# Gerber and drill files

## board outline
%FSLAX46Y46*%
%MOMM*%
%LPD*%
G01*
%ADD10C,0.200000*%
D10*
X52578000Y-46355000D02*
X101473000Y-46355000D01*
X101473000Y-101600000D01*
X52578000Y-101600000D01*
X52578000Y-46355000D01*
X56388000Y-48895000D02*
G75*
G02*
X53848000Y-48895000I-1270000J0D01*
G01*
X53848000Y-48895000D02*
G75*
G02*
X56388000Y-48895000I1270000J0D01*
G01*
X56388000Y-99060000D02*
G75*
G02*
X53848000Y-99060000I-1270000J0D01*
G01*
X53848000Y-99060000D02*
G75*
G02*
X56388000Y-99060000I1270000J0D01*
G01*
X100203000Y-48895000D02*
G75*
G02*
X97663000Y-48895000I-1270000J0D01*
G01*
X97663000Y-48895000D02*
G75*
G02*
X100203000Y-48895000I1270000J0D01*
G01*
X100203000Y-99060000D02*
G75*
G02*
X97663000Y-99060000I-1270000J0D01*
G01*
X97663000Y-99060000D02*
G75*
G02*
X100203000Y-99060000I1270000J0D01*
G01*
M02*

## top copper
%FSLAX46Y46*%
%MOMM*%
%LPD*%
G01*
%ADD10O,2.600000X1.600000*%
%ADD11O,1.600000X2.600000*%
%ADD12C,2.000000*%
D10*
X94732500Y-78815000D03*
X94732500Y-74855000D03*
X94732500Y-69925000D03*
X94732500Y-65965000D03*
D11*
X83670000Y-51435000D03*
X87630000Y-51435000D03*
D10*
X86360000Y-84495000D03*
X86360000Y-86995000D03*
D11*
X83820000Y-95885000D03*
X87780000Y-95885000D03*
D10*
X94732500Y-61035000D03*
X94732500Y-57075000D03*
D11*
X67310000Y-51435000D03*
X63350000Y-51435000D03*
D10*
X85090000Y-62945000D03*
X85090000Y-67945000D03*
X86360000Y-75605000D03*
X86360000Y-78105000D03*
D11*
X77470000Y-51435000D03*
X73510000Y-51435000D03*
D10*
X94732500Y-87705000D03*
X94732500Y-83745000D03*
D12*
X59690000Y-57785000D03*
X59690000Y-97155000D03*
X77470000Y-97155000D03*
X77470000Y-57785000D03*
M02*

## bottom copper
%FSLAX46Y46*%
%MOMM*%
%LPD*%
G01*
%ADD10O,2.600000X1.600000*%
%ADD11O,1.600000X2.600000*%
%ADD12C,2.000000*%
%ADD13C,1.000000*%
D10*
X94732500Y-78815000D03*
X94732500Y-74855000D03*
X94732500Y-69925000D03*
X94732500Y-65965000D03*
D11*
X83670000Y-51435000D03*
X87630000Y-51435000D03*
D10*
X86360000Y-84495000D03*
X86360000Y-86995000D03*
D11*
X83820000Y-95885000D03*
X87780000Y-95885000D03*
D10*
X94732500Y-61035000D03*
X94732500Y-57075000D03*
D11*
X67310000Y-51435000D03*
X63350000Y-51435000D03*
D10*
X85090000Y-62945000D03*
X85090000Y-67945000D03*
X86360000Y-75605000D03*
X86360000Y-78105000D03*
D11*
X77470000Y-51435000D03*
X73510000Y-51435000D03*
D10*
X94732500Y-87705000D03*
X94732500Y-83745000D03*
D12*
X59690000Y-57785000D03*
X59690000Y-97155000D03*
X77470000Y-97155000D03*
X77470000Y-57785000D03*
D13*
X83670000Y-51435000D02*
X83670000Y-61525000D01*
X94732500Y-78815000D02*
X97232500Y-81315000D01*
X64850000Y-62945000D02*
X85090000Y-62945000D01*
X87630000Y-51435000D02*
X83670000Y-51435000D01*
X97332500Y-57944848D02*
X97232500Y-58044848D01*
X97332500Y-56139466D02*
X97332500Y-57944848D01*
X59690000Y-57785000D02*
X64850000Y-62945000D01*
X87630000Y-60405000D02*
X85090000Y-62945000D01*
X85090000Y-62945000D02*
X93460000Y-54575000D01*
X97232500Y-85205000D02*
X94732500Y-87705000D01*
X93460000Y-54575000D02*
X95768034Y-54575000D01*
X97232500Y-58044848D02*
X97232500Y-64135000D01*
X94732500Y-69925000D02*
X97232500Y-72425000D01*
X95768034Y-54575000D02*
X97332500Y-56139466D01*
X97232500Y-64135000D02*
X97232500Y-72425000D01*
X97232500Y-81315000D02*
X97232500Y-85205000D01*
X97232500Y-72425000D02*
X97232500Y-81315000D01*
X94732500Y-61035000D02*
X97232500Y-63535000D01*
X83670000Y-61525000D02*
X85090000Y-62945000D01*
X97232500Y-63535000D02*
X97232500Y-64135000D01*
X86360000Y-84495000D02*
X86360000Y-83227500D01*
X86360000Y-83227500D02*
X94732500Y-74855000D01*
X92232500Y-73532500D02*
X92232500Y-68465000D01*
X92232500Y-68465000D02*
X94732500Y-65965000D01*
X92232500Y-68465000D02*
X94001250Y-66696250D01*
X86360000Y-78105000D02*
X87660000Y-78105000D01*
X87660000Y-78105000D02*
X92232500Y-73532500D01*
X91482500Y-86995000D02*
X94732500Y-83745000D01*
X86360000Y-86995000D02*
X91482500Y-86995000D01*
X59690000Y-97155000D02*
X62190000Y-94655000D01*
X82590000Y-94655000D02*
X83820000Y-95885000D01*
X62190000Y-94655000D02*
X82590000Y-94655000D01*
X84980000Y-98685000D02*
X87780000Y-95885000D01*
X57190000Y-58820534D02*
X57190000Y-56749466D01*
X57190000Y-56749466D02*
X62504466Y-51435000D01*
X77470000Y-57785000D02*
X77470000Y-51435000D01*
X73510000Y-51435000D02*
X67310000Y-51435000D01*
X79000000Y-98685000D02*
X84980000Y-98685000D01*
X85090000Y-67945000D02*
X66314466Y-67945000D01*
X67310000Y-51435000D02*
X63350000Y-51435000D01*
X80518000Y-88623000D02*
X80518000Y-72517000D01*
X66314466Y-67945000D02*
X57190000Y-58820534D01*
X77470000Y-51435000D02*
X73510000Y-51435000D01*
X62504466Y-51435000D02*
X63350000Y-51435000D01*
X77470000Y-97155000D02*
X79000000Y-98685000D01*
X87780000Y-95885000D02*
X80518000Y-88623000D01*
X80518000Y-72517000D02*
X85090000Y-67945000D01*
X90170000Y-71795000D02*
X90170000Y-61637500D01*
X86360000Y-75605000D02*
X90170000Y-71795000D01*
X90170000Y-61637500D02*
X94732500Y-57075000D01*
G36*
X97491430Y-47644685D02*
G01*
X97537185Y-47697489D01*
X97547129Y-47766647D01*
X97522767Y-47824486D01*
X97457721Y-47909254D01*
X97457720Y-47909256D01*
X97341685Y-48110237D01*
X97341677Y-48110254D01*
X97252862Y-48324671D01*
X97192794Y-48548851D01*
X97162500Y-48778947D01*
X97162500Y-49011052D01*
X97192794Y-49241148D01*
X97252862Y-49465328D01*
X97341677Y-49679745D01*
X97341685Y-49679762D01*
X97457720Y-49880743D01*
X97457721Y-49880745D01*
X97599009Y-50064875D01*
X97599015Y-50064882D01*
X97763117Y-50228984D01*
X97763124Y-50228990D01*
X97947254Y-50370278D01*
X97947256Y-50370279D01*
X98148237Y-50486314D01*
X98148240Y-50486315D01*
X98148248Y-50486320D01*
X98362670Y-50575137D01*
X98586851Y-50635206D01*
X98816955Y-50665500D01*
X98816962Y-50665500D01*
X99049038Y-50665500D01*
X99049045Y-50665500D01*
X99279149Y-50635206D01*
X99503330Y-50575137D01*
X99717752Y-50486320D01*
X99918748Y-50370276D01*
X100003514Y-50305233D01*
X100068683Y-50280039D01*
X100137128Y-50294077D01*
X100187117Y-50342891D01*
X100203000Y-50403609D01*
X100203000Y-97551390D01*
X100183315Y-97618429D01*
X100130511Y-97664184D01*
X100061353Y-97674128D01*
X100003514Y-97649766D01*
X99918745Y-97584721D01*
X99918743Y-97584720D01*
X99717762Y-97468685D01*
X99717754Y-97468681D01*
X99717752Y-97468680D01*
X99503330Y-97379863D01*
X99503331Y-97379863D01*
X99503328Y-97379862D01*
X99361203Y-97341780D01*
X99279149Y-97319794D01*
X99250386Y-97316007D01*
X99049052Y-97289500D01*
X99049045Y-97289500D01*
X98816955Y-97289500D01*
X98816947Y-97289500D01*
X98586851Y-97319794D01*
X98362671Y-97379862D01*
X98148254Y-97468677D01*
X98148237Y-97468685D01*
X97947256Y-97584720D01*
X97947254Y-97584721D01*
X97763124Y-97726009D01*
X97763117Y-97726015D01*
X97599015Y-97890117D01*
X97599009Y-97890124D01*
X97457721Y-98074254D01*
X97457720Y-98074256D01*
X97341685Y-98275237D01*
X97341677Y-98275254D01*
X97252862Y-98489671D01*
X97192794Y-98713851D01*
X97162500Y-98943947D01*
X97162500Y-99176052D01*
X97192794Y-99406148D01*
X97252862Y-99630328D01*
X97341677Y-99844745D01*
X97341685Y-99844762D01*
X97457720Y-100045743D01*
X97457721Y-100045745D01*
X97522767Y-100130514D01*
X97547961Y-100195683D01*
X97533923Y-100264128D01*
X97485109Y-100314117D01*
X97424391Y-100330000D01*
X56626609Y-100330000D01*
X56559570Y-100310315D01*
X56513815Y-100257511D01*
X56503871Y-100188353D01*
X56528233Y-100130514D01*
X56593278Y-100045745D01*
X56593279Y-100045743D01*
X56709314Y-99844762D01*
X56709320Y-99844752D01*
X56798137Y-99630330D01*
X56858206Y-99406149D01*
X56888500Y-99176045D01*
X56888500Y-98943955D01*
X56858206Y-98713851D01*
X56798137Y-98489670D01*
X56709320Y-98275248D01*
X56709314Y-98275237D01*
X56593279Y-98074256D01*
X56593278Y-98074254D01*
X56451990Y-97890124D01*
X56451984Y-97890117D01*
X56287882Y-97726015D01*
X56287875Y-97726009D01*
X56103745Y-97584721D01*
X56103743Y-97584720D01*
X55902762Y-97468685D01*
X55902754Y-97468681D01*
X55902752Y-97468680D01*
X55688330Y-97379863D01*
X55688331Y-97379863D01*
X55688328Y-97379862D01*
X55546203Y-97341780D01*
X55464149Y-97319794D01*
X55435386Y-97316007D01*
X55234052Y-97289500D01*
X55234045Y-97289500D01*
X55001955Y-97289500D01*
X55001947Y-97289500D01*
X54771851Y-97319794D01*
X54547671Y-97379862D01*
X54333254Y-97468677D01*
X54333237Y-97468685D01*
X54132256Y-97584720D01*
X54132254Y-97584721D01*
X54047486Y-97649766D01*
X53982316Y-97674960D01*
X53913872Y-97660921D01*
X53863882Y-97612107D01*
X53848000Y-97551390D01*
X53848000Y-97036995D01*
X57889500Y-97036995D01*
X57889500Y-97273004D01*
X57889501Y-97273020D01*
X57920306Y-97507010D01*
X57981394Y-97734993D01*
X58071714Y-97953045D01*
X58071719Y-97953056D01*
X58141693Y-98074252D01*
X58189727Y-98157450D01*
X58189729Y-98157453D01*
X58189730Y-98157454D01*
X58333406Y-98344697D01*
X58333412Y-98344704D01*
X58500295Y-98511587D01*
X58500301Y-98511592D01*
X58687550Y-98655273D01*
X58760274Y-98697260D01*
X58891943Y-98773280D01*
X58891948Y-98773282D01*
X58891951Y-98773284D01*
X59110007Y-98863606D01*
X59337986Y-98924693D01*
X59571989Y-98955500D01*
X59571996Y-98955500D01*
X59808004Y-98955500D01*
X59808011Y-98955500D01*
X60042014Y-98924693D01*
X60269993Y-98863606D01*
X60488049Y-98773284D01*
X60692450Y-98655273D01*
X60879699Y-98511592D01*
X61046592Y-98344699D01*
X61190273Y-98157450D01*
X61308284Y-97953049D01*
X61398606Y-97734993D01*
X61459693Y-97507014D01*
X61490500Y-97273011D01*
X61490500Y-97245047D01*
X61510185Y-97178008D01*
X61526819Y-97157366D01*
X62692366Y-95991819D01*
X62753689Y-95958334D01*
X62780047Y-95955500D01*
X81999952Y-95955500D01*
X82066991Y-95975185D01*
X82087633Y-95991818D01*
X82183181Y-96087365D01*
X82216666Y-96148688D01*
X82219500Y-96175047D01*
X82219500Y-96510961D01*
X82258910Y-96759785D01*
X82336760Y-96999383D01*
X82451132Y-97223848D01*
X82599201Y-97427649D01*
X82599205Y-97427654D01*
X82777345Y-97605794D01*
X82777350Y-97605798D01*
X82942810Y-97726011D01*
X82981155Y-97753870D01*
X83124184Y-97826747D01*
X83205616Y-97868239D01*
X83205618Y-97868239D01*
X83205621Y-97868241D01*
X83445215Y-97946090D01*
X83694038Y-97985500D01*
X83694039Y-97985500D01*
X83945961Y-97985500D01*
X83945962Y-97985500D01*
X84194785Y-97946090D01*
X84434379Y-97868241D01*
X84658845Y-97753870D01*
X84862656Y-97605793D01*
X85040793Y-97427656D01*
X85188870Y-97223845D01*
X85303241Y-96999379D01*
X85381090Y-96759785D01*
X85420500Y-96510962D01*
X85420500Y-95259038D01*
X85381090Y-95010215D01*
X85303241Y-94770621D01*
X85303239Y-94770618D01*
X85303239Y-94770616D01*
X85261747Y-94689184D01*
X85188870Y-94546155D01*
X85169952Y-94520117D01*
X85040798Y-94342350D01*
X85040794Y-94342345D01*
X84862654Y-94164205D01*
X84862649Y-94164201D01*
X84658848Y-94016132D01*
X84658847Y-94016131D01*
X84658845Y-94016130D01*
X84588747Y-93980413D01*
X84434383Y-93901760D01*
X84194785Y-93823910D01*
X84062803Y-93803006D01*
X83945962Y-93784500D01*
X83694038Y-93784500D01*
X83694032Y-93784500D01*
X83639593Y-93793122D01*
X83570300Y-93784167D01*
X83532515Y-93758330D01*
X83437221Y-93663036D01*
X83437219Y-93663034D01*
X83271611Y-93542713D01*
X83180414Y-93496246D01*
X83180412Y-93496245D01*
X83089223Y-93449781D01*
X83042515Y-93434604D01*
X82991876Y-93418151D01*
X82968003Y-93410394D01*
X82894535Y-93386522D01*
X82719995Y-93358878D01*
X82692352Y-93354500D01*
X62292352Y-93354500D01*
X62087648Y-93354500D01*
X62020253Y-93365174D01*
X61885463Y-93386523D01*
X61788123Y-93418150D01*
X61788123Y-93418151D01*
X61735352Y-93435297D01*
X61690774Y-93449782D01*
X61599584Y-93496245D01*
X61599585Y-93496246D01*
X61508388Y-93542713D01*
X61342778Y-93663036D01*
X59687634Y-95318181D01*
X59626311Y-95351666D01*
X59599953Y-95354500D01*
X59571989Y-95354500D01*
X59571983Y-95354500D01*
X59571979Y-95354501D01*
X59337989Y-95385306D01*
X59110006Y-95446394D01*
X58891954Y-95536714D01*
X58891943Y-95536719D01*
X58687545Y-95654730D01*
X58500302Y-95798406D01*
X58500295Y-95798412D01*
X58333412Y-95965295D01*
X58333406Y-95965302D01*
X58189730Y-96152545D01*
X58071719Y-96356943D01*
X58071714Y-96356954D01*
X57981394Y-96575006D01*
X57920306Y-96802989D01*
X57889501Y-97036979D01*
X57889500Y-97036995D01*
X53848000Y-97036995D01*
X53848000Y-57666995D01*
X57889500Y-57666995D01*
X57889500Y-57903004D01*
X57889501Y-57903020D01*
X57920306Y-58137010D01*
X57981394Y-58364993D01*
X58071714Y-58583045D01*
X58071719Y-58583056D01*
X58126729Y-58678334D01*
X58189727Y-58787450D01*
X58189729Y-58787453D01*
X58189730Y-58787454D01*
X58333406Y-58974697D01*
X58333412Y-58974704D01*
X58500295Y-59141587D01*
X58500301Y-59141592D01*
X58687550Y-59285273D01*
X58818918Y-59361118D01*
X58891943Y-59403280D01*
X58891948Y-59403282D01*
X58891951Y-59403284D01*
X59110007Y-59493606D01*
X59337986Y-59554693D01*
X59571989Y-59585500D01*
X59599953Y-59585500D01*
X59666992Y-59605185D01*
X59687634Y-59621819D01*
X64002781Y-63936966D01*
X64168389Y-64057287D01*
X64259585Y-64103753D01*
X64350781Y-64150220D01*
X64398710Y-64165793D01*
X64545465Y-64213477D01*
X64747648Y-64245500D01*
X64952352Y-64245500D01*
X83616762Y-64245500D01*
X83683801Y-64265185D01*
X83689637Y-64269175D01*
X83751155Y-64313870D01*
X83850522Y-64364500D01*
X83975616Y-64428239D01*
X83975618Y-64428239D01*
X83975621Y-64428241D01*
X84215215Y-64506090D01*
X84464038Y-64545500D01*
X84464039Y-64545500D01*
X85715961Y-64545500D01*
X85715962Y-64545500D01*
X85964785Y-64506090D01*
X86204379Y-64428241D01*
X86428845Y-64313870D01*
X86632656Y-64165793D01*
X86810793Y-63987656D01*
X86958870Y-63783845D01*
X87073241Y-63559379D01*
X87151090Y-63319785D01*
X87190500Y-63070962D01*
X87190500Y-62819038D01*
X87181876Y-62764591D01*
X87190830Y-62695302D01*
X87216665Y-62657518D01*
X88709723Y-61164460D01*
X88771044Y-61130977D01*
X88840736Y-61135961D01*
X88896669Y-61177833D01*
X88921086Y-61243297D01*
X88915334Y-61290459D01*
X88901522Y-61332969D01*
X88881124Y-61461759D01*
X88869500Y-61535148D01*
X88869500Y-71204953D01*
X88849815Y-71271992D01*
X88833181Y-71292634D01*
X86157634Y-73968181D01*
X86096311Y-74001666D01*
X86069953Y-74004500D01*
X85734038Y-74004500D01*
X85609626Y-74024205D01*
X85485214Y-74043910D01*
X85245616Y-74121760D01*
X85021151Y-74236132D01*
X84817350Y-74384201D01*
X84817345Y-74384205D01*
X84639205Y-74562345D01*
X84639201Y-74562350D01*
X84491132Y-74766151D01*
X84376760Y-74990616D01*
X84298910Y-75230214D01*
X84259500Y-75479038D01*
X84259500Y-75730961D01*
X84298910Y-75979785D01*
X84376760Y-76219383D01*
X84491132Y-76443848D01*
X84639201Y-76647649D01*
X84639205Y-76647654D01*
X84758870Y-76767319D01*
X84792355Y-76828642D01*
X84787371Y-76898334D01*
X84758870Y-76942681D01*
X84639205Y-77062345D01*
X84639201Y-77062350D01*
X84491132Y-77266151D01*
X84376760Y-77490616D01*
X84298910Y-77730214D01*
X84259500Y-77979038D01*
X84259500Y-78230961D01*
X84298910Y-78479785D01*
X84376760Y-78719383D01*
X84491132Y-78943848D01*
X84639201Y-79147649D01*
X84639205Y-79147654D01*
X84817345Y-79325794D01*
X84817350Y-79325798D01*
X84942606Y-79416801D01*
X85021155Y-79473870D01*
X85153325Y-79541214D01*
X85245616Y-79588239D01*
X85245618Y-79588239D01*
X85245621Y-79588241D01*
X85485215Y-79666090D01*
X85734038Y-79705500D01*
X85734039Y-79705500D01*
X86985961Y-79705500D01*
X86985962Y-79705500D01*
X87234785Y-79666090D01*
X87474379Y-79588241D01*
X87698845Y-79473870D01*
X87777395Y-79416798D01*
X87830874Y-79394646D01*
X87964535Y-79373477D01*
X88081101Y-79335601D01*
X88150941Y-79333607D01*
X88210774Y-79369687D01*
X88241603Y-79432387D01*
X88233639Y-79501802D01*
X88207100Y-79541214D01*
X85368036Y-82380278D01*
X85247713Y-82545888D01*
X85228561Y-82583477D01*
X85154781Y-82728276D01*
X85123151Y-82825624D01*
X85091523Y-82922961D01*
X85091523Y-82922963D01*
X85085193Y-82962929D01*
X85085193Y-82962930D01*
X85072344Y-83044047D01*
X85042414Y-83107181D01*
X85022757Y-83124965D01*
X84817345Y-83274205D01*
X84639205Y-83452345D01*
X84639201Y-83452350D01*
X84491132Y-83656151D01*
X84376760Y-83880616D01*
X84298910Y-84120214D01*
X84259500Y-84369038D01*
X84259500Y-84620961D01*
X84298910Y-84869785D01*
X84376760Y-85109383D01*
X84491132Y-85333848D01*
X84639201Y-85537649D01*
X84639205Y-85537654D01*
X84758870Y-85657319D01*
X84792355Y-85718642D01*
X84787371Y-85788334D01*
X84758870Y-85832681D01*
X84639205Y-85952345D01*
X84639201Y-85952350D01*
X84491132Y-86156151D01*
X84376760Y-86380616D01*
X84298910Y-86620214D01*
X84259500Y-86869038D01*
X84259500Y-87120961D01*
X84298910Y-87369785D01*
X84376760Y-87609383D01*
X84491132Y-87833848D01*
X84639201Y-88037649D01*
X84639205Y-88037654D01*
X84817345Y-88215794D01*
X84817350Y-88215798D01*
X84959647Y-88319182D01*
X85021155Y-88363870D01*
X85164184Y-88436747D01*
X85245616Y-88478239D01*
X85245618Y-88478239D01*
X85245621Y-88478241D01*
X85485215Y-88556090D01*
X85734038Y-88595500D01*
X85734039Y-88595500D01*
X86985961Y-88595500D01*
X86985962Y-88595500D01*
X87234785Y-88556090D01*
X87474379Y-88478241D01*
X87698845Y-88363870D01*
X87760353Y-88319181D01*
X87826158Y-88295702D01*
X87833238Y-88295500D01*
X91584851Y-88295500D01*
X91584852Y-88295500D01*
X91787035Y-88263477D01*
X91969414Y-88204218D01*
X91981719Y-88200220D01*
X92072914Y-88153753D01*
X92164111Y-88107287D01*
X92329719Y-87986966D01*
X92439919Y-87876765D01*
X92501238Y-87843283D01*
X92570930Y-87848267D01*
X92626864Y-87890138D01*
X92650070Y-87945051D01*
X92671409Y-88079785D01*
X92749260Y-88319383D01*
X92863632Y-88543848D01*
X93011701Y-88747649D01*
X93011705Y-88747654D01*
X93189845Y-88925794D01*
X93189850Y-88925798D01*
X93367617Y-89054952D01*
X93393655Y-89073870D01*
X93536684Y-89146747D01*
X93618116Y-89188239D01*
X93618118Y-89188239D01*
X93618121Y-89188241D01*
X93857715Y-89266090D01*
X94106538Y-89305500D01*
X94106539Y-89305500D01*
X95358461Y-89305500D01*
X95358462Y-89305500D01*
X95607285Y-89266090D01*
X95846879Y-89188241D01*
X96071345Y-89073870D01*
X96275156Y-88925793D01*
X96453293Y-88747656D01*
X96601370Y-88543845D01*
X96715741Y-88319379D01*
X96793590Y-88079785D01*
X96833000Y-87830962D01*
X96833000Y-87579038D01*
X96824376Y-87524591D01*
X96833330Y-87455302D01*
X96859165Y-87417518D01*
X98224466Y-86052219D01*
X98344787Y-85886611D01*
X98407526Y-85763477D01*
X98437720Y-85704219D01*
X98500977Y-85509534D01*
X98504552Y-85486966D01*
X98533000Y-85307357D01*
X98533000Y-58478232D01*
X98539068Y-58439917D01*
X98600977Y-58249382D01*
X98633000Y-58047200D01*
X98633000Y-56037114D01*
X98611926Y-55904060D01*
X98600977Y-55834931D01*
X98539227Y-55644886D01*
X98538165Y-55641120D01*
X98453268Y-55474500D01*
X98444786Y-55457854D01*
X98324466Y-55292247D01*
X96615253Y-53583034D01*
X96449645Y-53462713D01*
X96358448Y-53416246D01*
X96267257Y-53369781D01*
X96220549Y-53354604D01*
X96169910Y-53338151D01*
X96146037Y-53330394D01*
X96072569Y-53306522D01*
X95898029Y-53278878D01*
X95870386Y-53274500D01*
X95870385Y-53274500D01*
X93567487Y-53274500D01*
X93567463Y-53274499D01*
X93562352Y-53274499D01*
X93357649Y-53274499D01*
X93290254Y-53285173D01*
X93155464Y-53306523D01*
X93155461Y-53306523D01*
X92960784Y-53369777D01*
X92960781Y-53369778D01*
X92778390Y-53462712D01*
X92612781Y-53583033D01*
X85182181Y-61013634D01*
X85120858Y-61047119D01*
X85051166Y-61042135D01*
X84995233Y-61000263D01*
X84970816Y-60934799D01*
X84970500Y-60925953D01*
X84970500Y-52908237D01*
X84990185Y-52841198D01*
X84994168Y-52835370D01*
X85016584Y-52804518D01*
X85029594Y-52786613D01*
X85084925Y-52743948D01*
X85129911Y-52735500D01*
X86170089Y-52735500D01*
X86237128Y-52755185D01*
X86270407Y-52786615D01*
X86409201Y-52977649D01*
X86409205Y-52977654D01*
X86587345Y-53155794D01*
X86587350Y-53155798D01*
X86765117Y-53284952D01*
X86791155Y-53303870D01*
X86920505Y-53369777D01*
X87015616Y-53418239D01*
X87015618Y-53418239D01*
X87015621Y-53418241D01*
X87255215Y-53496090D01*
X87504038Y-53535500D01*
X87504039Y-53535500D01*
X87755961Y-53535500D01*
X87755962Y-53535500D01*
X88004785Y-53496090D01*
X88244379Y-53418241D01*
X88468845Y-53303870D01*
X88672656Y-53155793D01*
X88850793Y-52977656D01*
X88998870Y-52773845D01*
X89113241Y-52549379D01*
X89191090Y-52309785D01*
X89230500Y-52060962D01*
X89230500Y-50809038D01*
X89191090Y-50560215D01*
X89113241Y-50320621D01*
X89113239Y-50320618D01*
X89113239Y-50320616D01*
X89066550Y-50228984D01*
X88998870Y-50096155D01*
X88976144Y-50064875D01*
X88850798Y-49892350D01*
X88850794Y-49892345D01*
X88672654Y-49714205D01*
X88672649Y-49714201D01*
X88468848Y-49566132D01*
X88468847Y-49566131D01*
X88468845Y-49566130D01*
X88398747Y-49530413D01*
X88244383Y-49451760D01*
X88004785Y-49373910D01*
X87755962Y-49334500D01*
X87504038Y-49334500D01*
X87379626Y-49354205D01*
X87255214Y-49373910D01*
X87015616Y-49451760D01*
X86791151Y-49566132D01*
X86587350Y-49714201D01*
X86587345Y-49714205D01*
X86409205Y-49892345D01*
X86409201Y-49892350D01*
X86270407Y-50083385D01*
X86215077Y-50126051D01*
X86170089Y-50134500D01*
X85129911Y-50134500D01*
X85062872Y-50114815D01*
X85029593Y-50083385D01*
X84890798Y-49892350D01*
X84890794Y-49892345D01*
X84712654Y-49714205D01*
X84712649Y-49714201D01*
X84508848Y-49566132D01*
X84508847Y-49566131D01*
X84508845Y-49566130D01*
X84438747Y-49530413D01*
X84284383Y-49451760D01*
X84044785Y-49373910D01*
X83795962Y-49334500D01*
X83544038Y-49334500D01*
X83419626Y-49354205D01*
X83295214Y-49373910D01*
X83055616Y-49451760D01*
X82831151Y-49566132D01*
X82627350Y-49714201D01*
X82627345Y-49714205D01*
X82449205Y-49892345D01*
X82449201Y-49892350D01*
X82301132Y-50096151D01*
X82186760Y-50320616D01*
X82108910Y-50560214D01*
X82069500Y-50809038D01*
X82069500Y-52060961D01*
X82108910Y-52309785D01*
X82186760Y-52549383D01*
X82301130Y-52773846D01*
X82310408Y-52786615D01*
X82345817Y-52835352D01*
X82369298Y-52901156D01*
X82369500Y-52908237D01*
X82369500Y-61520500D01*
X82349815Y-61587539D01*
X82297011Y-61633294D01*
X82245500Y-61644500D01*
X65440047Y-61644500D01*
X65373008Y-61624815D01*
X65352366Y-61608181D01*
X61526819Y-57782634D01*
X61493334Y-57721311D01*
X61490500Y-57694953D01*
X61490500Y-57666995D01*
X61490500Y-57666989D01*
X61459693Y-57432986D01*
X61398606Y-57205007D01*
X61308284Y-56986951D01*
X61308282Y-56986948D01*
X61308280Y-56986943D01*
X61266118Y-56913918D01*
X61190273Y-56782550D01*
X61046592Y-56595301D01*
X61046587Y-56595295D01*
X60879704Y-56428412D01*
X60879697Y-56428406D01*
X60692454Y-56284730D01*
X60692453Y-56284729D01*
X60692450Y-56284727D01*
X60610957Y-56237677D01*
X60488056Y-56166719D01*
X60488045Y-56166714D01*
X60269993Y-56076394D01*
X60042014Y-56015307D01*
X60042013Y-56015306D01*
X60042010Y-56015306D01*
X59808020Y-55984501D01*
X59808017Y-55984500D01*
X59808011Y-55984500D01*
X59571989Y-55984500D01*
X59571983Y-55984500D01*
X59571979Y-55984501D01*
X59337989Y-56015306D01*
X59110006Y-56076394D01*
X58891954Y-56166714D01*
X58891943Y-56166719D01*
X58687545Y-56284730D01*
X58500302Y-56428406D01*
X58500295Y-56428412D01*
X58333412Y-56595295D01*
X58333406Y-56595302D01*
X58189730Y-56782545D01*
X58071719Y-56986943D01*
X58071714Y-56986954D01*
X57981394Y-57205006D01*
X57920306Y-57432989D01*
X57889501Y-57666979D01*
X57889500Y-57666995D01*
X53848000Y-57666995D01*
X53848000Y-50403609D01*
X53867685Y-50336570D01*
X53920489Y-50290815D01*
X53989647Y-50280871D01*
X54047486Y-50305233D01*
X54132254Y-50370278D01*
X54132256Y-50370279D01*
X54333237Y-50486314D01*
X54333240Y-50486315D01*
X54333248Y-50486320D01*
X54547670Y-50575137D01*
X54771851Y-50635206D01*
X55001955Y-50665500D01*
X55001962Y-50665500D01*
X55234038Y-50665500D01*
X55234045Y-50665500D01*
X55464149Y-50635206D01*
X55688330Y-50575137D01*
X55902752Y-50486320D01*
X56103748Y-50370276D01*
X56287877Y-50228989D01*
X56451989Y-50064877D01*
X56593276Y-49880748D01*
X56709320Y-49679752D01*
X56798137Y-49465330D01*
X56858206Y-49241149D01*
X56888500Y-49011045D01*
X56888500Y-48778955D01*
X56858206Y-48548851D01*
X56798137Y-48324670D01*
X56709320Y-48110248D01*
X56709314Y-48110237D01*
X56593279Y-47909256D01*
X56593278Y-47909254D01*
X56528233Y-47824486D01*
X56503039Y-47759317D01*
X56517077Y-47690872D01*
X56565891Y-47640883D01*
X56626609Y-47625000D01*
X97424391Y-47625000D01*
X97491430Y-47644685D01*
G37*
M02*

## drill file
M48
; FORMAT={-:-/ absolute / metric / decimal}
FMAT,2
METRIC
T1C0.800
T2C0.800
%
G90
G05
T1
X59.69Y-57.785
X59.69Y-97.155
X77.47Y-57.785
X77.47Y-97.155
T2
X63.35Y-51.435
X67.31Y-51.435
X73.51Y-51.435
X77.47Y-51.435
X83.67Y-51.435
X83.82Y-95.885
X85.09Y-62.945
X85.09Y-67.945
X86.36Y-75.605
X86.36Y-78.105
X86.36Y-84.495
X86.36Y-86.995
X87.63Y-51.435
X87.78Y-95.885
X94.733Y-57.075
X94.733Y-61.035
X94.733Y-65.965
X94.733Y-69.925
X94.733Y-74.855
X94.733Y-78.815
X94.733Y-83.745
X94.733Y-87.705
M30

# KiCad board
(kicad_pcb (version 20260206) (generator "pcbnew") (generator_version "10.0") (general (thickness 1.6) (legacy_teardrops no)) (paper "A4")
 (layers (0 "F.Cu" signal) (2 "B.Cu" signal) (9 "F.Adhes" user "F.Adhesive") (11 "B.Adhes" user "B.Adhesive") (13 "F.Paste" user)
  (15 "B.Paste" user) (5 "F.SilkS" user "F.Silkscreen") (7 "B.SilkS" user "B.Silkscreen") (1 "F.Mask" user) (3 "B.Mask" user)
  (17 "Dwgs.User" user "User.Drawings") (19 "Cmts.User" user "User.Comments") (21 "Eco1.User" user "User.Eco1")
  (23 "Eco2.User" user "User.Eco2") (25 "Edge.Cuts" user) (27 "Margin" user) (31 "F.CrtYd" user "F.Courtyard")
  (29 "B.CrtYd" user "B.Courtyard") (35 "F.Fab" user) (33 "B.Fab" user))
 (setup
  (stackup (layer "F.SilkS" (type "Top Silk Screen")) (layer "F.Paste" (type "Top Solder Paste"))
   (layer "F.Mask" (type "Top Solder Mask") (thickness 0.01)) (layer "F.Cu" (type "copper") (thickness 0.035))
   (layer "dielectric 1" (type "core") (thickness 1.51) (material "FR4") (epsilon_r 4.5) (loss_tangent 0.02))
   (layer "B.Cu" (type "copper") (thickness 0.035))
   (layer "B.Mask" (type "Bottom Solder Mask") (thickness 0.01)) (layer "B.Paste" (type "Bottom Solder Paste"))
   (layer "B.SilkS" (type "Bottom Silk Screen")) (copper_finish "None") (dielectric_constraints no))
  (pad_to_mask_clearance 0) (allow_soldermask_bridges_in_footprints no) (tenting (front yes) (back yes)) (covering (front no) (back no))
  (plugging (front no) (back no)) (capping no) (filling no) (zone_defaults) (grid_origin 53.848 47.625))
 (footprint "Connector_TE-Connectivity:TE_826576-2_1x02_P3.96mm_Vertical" (layer "F.Cu") (at 94.7325 78.815 90)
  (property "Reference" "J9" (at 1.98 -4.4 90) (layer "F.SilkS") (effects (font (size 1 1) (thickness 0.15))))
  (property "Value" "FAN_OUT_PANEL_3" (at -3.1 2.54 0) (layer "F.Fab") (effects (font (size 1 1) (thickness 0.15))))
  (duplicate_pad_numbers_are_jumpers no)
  (pad "1" thru_hole oval (at 0 0 180) (size 2.6 1.6) (drill 0.8) (layers "*.Cu" "*.Mask") (remove_unused_layers yes) (keep_end_layers yes)
   (zone_layer_connections) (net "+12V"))
  (pad "2" thru_hole oval (at 3.96 0 180) (size 2.6 1.6) (drill 0.8) (layers "*.Cu" "*.Mask") (remove_unused_layers yes)
   (keep_end_layers yes) (zone_layer_connections) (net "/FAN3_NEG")))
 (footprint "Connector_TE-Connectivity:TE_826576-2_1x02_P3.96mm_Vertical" (layer "F.Cu") (at 94.7325 69.925 90)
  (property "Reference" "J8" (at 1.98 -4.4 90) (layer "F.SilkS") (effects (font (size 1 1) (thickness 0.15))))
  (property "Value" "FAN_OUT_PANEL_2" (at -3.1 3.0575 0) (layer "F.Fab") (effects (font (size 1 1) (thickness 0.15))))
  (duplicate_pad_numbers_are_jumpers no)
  (pad "1" thru_hole oval (at 0 0 180) (size 2.6 1.6) (drill 0.8) (layers "*.Cu" "*.Mask") (remove_unused_layers yes) (keep_end_layers yes)
   (zone_layer_connections) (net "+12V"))
  (pad "2" thru_hole oval (at 3.96 0 180) (size 2.6 1.6) (drill 0.8) (layers "*.Cu" "*.Mask") (remove_unused_layers yes)
   (keep_end_layers yes) (zone_layer_connections) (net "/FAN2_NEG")))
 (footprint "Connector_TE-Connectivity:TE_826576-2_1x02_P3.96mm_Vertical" (layer "F.Cu") (at 83.67 51.435)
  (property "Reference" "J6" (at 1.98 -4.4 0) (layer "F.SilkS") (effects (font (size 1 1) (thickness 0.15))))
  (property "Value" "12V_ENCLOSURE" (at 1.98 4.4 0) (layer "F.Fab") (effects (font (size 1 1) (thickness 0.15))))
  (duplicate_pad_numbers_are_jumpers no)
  (pad "1" thru_hole oval (at 0 0 90) (size 2.6 1.6) (drill 0.8) (layers "*.Cu" "*.Mask") (remove_unused_layers yes) (keep_end_layers yes)
   (zone_layer_connections) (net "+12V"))
  (pad "2" thru_hole oval (at 3.96 0 90) (size 2.6 1.6) (drill 0.8) (layers "*.Cu" "*.Mask") (remove_unused_layers yes)
   (keep_end_layers yes) (zone_layer_connections) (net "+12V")))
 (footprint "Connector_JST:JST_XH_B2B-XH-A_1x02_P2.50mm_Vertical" (layer "F.Cu") (at 86.36 84.495 -90)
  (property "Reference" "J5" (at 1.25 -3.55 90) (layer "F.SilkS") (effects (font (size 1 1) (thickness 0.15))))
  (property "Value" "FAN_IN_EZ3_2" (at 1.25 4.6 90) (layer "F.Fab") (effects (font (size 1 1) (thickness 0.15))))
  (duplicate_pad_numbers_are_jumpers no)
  (pad "1" thru_hole oval (at 0 0) (size 2.6 1.6) (drill 0.8) (layers "*.Cu" "*.Mask") (remove_unused_layers yes) (keep_end_layers yes)
   (zone_layer_connections) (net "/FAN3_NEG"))
  (pad "2" thru_hole oval (at 2.5 0) (size 2.6 1.6) (drill 0.8) (layers "*.Cu" "*.Mask") (remove_unused_layers yes) (keep_end_layers yes)
   (zone_layer_connections) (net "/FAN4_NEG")))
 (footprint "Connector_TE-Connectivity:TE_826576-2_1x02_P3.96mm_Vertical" (layer "F.Cu") (at 83.82 95.885)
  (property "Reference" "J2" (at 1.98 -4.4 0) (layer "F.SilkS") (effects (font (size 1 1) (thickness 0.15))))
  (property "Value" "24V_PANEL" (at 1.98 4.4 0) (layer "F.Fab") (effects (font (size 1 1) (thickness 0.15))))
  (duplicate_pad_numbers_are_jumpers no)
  (pad "1" thru_hole oval (at 0 0 90) (size 2.6 1.6) (drill 0.8) (layers "*.Cu" "*.Mask") (remove_unused_layers yes) (keep_end_layers yes)
   (zone_layer_connections) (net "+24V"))
  (pad "2" thru_hole oval (at 3.96 0 90) (size 2.6 1.6) (drill 0.8) (layers "*.Cu" "*.Mask") (remove_unused_layers yes)
   (keep_end_layers yes) (zone_layer_connections) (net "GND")))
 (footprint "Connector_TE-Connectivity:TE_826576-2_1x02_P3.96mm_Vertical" (layer "F.Cu") (at 94.7325 61.035 90)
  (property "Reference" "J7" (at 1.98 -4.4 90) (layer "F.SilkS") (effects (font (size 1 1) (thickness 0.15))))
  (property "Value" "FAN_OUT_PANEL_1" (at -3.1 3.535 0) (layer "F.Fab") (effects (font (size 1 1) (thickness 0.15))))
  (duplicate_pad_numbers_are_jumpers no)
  (pad "1" thru_hole oval (at 0 0 180) (size 2.6 1.6) (drill 0.8) (layers "*.Cu" "*.Mask") (remove_unused_layers yes) (keep_end_layers yes)
   (zone_layer_connections) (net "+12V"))
  (pad "2" thru_hole oval (at 3.96 0 180) (size 2.6 1.6) (drill 0.8) (layers "*.Cu" "*.Mask") (remove_unused_layers yes)
   (keep_end_layers yes) (zone_layer_connections) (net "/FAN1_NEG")))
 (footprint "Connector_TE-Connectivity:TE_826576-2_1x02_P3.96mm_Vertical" (layer "F.Cu") (at 67.31 51.435 180)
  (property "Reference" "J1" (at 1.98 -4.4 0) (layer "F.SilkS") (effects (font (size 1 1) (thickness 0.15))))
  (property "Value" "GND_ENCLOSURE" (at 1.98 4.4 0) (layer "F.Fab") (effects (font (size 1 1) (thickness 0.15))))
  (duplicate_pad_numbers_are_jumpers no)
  (pad "1" thru_hole oval (at 0 0 270) (size 2.6 1.6) (drill 0.8) (layers "*.Cu" "*.Mask") (remove_unused_layers yes) (keep_end_layers yes)
   (zone_layer_connections) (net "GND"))
  (pad "2" thru_hole oval (at 3.96 0 270) (size 2.6 1.6) (drill 0.8) (layers "*.Cu" "*.Mask") (remove_unused_layers yes)
   (keep_end_layers yes) (zone_layer_connections) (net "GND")))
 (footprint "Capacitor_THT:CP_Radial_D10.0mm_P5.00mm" (layer "F.Cu") (at 85.09 62.945 -90)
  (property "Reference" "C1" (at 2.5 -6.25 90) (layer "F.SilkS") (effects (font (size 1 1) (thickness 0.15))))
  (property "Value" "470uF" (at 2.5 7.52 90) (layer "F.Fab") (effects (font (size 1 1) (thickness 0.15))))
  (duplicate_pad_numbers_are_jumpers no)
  (pad "1" thru_hole oval (at 0 0) (size 2.6 1.6) (drill 0.8) (layers "*.Cu" "*.Mask") (remove_unused_layers yes) (keep_end_layers yes)
   (zone_layer_connections) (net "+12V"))
  (pad "2" thru_hole oval (at 5 0) (size 2.6 1.6) (drill 0.8) (layers "*.Cu" "*.Mask") (remove_unused_layers yes) (keep_end_layers yes)
   (zone_layer_connections) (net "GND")))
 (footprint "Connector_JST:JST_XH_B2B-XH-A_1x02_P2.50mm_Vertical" (layer "F.Cu") (at 86.36 75.605 -90)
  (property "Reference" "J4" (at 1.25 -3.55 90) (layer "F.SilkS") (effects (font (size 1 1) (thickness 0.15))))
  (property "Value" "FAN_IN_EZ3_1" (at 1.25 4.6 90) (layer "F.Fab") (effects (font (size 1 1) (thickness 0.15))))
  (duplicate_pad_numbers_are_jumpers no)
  (pad "1" thru_hole oval (at 0 0) (size 2.6 1.6) (drill 0.8) (layers "*.Cu" "*.Mask") (remove_unused_layers yes) (keep_end_layers yes)
   (zone_layer_connections) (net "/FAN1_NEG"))
  (pad "2" thru_hole oval (at 2.5 0) (size 2.6 1.6) (drill 0.8) (layers "*.Cu" "*.Mask") (remove_unused_layers yes) (keep_end_layers yes)
   (zone_layer_connections) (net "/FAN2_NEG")))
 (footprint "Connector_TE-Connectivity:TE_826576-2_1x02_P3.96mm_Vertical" (layer "F.Cu") (at 77.47 51.435 180)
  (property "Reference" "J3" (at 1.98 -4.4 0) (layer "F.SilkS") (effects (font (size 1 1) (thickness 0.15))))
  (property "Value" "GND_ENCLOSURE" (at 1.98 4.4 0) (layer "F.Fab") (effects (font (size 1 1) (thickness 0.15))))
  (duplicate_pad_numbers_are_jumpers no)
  (pad "1" thru_hole oval (at 0 0 270) (size 2.6 1.6) (drill 0.8) (layers "*.Cu" "*.Mask") (remove_unused_layers yes) (keep_end_layers yes)
   (zone_layer_connections) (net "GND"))
  (pad "2" thru_hole oval (at 3.96 0 270) (size 2.6 1.6) (drill 0.8) (layers "*.Cu" "*.Mask") (remove_unused_layers yes)
   (keep_end_layers yes) (zone_layer_connections) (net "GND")))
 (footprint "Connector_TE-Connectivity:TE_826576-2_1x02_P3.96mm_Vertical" (layer "F.Cu") (at 94.7325 87.705 90)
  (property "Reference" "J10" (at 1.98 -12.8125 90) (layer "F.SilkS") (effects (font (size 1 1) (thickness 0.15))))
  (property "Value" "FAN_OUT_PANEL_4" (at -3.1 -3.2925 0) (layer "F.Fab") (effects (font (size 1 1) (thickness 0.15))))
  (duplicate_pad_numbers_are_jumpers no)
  (pad "1" thru_hole oval (at 0 0 180) (size 2.6 1.6) (drill 0.8) (layers "*.Cu" "*.Mask") (remove_unused_layers yes) (keep_end_layers yes)
   (zone_layer_connections) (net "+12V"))
  (pad "2" thru_hole oval (at 3.96 0 180) (size 2.6 1.6) (drill 0.8) (layers "*.Cu" "*.Mask") (remove_unused_layers yes)
   (keep_end_layers yes) (zone_layer_connections) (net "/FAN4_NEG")))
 (gr_rect (start 52.578 46.355) (end 101.473 101.6) (stroke (width 0.2) (type solid)) (fill no) (layer "Edge.Cuts"))
 (gr_circle (center 55.118 48.895) (end 56.388 48.895) (stroke (width 0.2) (type solid)) (fill no) (layer "Edge.Cuts"))
 (gr_circle (center 55.118 99.06) (end 56.388 99.06) (stroke (width 0.2) (type solid)) (fill no) (layer "Edge.Cuts"))
 (gr_circle (center 98.933 48.895) (end 100.203 48.895) (stroke (width 0.2) (type solid)) (fill no) (layer "Edge.Cuts"))
 (gr_circle (center 98.933 99.06) (end 100.203 99.06) (stroke (width 0.2) (type solid)) (fill no) (layer "Edge.Cuts"))
 (via (at 59.69 57.785) (size 2) (drill 0.8) (layers "F.Cu" "B.Cu") (free yes) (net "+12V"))
 (segment (start 83.67 51.435) (end 83.67 61.525) (width 1) (layer "B.Cu") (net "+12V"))
 (segment (start 94.7325 78.815) (end 97.2325 81.315) (width 1) (layer "B.Cu") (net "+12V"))
 (segment (start 64.85 62.945) (end 85.09 62.945) (width 1) (layer "B.Cu") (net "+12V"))
 (segment (start 87.63 51.435) (end 83.67 51.435) (width 1) (layer "B.Cu") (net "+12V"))
 (segment (start 97.3325 57.944848) (end 97.2325 58.044848) (width 1) (layer "B.Cu") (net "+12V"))
 (segment (start 97.3325 56.139466) (end 97.3325 57.944848) (width 1) (layer "B.Cu") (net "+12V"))
 (segment (start 59.69 57.785) (end 64.85 62.945) (width 1) (layer "B.Cu") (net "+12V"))
 (segment (start 87.63 60.405) (end 85.09 62.945) (width 1) (layer "B.Cu") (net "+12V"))
 (segment (start 85.09 62.945) (end 93.46 54.575) (width 1) (layer "B.Cu") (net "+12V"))
 (segment (start 97.2325 85.205) (end 94.7325 87.705) (width 1) (layer "B.Cu") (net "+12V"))
 (segment (start 93.46 54.575) (end 95.768034 54.575) (width 1) (layer "B.Cu") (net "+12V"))
 (segment (start 97.2325 58.044848) (end 97.2325 64.135) (width 1) (layer "B.Cu") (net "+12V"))
 (segment (start 94.7325 69.925) (end 97.2325 72.425) (width 1) (layer "B.Cu") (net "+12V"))
 (segment (start 95.768034 54.575) (end 97.3325 56.139466) (width 1) (layer "B.Cu") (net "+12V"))
 (segment (start 97.2325 64.135) (end 97.2325 72.425) (width 1) (layer "B.Cu") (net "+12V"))
 (segment (start 97.2325 81.315) (end 97.2325 85.205) (width 1) (layer "B.Cu") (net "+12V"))
 (segment (start 97.2325 72.425) (end 97.2325 81.315) (width 1) (layer "B.Cu") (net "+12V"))
 (segment (start 94.7325 61.035) (end 97.2325 63.535) (width 1) (layer "B.Cu") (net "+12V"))
 (segment (start 83.67 61.525) (end 85.09 62.945) (width 1) (layer "B.Cu") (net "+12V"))
 (segment (start 97.2325 63.535) (end 97.2325 64.135) (width 1) (layer "B.Cu") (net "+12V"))
 (segment (start 86.36 84.495) (end 86.36 83.2275) (width 1) (layer "B.Cu") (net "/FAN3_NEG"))
 (segment (start 86.36 83.2275) (end 94.7325 74.855) (width 1) (layer "B.Cu") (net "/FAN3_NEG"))
 (segment (start 92.2325 73.5325) (end 92.2325 68.465) (width 1) (layer "B.Cu") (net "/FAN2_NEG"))
 (segment (start 92.2325 68.465) (end 94.7325 65.965) (width 1) (layer "B.Cu") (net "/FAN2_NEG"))
 (segment (start 92.2325 68.465) (end 94.00125 66.69625) (width 1) (layer "B.Cu") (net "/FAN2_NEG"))
 (segment (start 86.36 78.105) (end 87.66 78.105) (width 1) (layer "B.Cu") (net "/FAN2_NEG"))
 (segment (start 87.66 78.105) (end 92.2325 73.5325) (width 1) (layer "B.Cu") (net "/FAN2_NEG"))
 (segment (start 91.4825 86.995) (end 94.7325 83.745) (width 1) (layer "B.Cu") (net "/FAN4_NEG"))
 (segment (start 86.36 86.995) (end 91.4825 86.995) (width 1) (layer "B.Cu") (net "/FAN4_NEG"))
 (via (at 59.69 97.155) (size 2) (drill 0.8) (layers "F.Cu" "B.Cu") (free yes) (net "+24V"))
 (segment (start 59.69 97.155) (end 62.19 94.655) (width 1) (layer "B.Cu") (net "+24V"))
 (segment (start 82.59 94.655) (end 83.82 95.885) (width 1) (layer "B.Cu") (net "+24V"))
 (segment (start 62.19 94.655) (end 82.59 94.655) (width 1) (layer "B.Cu") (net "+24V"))
 (via (at 77.47 97.155) (size 2) (drill 0.8) (layers "F.Cu" "B.Cu") (free yes) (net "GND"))
 (via (at 77.47 57.785) (size 2) (drill 0.8) (layers "F.Cu" "B.Cu") (free yes) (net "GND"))
 (segment (start 84.98 98.685) (end 87.78 95.885) (width 1) (layer "B.Cu") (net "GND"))
 (segment (start 57.19 58.820534) (end 57.19 56.749466) (width 1) (layer "B.Cu") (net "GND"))
 (segment (start 57.19 56.749466) (end 62.504466 51.435) (width 1) (layer "B.Cu") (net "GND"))
 (segment (start 77.47 57.785) (end 77.47 51.435) (width 1) (layer "B.Cu") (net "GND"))
 (segment (start 73.51 51.435) (end 67.31 51.435) (width 1) (layer "B.Cu") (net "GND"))
 (segment (start 79 98.685) (end 84.98 98.685) (width 1) (layer "B.Cu") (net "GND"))
 (segment (start 85.09 67.945) (end 66.314466 67.945) (width 1) (layer "B.Cu") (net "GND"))
 (segment (start 67.31 51.435) (end 63.35 51.435) (width 1) (layer "B.Cu") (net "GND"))
 (segment (start 80.518 88.623) (end 80.518 72.517) (width 1) (layer "B.Cu") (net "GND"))
 (segment (start 66.314466 67.945) (end 57.19 58.820534) (width 1) (layer "B.Cu") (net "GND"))
 (segment (start 77.47 51.435) (end 73.51 51.435) (width 1) (layer "B.Cu") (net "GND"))
 (segment (start 62.504466 51.435) (end 63.35 51.435) (width 1) (layer "B.Cu") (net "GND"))
 (segment (start 77.47 97.155) (end 79 98.685) (width 1) (layer "B.Cu") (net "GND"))
 (segment (start 87.78 95.885) (end 80.518 88.623) (width 1) (layer "B.Cu") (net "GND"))
 (segment (start 80.518 72.517) (end 85.09 67.945) (width 1) (layer "B.Cu") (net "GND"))
 (segment (start 90.17 71.795) (end 90.17 61.6375) (width 1) (layer "B.Cu") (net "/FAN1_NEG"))
 (segment (start 86.36 75.605) (end 90.17 71.795) (width 1) (layer "B.Cu") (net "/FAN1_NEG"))
 (segment (start 90.17 61.6375) (end 94.7325 57.075) (width 1) (layer "B.Cu") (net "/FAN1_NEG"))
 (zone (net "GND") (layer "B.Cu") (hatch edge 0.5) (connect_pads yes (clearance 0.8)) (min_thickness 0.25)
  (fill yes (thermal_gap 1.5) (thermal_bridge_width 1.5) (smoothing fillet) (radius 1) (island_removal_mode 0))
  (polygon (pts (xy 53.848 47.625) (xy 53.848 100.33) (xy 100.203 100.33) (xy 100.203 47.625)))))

